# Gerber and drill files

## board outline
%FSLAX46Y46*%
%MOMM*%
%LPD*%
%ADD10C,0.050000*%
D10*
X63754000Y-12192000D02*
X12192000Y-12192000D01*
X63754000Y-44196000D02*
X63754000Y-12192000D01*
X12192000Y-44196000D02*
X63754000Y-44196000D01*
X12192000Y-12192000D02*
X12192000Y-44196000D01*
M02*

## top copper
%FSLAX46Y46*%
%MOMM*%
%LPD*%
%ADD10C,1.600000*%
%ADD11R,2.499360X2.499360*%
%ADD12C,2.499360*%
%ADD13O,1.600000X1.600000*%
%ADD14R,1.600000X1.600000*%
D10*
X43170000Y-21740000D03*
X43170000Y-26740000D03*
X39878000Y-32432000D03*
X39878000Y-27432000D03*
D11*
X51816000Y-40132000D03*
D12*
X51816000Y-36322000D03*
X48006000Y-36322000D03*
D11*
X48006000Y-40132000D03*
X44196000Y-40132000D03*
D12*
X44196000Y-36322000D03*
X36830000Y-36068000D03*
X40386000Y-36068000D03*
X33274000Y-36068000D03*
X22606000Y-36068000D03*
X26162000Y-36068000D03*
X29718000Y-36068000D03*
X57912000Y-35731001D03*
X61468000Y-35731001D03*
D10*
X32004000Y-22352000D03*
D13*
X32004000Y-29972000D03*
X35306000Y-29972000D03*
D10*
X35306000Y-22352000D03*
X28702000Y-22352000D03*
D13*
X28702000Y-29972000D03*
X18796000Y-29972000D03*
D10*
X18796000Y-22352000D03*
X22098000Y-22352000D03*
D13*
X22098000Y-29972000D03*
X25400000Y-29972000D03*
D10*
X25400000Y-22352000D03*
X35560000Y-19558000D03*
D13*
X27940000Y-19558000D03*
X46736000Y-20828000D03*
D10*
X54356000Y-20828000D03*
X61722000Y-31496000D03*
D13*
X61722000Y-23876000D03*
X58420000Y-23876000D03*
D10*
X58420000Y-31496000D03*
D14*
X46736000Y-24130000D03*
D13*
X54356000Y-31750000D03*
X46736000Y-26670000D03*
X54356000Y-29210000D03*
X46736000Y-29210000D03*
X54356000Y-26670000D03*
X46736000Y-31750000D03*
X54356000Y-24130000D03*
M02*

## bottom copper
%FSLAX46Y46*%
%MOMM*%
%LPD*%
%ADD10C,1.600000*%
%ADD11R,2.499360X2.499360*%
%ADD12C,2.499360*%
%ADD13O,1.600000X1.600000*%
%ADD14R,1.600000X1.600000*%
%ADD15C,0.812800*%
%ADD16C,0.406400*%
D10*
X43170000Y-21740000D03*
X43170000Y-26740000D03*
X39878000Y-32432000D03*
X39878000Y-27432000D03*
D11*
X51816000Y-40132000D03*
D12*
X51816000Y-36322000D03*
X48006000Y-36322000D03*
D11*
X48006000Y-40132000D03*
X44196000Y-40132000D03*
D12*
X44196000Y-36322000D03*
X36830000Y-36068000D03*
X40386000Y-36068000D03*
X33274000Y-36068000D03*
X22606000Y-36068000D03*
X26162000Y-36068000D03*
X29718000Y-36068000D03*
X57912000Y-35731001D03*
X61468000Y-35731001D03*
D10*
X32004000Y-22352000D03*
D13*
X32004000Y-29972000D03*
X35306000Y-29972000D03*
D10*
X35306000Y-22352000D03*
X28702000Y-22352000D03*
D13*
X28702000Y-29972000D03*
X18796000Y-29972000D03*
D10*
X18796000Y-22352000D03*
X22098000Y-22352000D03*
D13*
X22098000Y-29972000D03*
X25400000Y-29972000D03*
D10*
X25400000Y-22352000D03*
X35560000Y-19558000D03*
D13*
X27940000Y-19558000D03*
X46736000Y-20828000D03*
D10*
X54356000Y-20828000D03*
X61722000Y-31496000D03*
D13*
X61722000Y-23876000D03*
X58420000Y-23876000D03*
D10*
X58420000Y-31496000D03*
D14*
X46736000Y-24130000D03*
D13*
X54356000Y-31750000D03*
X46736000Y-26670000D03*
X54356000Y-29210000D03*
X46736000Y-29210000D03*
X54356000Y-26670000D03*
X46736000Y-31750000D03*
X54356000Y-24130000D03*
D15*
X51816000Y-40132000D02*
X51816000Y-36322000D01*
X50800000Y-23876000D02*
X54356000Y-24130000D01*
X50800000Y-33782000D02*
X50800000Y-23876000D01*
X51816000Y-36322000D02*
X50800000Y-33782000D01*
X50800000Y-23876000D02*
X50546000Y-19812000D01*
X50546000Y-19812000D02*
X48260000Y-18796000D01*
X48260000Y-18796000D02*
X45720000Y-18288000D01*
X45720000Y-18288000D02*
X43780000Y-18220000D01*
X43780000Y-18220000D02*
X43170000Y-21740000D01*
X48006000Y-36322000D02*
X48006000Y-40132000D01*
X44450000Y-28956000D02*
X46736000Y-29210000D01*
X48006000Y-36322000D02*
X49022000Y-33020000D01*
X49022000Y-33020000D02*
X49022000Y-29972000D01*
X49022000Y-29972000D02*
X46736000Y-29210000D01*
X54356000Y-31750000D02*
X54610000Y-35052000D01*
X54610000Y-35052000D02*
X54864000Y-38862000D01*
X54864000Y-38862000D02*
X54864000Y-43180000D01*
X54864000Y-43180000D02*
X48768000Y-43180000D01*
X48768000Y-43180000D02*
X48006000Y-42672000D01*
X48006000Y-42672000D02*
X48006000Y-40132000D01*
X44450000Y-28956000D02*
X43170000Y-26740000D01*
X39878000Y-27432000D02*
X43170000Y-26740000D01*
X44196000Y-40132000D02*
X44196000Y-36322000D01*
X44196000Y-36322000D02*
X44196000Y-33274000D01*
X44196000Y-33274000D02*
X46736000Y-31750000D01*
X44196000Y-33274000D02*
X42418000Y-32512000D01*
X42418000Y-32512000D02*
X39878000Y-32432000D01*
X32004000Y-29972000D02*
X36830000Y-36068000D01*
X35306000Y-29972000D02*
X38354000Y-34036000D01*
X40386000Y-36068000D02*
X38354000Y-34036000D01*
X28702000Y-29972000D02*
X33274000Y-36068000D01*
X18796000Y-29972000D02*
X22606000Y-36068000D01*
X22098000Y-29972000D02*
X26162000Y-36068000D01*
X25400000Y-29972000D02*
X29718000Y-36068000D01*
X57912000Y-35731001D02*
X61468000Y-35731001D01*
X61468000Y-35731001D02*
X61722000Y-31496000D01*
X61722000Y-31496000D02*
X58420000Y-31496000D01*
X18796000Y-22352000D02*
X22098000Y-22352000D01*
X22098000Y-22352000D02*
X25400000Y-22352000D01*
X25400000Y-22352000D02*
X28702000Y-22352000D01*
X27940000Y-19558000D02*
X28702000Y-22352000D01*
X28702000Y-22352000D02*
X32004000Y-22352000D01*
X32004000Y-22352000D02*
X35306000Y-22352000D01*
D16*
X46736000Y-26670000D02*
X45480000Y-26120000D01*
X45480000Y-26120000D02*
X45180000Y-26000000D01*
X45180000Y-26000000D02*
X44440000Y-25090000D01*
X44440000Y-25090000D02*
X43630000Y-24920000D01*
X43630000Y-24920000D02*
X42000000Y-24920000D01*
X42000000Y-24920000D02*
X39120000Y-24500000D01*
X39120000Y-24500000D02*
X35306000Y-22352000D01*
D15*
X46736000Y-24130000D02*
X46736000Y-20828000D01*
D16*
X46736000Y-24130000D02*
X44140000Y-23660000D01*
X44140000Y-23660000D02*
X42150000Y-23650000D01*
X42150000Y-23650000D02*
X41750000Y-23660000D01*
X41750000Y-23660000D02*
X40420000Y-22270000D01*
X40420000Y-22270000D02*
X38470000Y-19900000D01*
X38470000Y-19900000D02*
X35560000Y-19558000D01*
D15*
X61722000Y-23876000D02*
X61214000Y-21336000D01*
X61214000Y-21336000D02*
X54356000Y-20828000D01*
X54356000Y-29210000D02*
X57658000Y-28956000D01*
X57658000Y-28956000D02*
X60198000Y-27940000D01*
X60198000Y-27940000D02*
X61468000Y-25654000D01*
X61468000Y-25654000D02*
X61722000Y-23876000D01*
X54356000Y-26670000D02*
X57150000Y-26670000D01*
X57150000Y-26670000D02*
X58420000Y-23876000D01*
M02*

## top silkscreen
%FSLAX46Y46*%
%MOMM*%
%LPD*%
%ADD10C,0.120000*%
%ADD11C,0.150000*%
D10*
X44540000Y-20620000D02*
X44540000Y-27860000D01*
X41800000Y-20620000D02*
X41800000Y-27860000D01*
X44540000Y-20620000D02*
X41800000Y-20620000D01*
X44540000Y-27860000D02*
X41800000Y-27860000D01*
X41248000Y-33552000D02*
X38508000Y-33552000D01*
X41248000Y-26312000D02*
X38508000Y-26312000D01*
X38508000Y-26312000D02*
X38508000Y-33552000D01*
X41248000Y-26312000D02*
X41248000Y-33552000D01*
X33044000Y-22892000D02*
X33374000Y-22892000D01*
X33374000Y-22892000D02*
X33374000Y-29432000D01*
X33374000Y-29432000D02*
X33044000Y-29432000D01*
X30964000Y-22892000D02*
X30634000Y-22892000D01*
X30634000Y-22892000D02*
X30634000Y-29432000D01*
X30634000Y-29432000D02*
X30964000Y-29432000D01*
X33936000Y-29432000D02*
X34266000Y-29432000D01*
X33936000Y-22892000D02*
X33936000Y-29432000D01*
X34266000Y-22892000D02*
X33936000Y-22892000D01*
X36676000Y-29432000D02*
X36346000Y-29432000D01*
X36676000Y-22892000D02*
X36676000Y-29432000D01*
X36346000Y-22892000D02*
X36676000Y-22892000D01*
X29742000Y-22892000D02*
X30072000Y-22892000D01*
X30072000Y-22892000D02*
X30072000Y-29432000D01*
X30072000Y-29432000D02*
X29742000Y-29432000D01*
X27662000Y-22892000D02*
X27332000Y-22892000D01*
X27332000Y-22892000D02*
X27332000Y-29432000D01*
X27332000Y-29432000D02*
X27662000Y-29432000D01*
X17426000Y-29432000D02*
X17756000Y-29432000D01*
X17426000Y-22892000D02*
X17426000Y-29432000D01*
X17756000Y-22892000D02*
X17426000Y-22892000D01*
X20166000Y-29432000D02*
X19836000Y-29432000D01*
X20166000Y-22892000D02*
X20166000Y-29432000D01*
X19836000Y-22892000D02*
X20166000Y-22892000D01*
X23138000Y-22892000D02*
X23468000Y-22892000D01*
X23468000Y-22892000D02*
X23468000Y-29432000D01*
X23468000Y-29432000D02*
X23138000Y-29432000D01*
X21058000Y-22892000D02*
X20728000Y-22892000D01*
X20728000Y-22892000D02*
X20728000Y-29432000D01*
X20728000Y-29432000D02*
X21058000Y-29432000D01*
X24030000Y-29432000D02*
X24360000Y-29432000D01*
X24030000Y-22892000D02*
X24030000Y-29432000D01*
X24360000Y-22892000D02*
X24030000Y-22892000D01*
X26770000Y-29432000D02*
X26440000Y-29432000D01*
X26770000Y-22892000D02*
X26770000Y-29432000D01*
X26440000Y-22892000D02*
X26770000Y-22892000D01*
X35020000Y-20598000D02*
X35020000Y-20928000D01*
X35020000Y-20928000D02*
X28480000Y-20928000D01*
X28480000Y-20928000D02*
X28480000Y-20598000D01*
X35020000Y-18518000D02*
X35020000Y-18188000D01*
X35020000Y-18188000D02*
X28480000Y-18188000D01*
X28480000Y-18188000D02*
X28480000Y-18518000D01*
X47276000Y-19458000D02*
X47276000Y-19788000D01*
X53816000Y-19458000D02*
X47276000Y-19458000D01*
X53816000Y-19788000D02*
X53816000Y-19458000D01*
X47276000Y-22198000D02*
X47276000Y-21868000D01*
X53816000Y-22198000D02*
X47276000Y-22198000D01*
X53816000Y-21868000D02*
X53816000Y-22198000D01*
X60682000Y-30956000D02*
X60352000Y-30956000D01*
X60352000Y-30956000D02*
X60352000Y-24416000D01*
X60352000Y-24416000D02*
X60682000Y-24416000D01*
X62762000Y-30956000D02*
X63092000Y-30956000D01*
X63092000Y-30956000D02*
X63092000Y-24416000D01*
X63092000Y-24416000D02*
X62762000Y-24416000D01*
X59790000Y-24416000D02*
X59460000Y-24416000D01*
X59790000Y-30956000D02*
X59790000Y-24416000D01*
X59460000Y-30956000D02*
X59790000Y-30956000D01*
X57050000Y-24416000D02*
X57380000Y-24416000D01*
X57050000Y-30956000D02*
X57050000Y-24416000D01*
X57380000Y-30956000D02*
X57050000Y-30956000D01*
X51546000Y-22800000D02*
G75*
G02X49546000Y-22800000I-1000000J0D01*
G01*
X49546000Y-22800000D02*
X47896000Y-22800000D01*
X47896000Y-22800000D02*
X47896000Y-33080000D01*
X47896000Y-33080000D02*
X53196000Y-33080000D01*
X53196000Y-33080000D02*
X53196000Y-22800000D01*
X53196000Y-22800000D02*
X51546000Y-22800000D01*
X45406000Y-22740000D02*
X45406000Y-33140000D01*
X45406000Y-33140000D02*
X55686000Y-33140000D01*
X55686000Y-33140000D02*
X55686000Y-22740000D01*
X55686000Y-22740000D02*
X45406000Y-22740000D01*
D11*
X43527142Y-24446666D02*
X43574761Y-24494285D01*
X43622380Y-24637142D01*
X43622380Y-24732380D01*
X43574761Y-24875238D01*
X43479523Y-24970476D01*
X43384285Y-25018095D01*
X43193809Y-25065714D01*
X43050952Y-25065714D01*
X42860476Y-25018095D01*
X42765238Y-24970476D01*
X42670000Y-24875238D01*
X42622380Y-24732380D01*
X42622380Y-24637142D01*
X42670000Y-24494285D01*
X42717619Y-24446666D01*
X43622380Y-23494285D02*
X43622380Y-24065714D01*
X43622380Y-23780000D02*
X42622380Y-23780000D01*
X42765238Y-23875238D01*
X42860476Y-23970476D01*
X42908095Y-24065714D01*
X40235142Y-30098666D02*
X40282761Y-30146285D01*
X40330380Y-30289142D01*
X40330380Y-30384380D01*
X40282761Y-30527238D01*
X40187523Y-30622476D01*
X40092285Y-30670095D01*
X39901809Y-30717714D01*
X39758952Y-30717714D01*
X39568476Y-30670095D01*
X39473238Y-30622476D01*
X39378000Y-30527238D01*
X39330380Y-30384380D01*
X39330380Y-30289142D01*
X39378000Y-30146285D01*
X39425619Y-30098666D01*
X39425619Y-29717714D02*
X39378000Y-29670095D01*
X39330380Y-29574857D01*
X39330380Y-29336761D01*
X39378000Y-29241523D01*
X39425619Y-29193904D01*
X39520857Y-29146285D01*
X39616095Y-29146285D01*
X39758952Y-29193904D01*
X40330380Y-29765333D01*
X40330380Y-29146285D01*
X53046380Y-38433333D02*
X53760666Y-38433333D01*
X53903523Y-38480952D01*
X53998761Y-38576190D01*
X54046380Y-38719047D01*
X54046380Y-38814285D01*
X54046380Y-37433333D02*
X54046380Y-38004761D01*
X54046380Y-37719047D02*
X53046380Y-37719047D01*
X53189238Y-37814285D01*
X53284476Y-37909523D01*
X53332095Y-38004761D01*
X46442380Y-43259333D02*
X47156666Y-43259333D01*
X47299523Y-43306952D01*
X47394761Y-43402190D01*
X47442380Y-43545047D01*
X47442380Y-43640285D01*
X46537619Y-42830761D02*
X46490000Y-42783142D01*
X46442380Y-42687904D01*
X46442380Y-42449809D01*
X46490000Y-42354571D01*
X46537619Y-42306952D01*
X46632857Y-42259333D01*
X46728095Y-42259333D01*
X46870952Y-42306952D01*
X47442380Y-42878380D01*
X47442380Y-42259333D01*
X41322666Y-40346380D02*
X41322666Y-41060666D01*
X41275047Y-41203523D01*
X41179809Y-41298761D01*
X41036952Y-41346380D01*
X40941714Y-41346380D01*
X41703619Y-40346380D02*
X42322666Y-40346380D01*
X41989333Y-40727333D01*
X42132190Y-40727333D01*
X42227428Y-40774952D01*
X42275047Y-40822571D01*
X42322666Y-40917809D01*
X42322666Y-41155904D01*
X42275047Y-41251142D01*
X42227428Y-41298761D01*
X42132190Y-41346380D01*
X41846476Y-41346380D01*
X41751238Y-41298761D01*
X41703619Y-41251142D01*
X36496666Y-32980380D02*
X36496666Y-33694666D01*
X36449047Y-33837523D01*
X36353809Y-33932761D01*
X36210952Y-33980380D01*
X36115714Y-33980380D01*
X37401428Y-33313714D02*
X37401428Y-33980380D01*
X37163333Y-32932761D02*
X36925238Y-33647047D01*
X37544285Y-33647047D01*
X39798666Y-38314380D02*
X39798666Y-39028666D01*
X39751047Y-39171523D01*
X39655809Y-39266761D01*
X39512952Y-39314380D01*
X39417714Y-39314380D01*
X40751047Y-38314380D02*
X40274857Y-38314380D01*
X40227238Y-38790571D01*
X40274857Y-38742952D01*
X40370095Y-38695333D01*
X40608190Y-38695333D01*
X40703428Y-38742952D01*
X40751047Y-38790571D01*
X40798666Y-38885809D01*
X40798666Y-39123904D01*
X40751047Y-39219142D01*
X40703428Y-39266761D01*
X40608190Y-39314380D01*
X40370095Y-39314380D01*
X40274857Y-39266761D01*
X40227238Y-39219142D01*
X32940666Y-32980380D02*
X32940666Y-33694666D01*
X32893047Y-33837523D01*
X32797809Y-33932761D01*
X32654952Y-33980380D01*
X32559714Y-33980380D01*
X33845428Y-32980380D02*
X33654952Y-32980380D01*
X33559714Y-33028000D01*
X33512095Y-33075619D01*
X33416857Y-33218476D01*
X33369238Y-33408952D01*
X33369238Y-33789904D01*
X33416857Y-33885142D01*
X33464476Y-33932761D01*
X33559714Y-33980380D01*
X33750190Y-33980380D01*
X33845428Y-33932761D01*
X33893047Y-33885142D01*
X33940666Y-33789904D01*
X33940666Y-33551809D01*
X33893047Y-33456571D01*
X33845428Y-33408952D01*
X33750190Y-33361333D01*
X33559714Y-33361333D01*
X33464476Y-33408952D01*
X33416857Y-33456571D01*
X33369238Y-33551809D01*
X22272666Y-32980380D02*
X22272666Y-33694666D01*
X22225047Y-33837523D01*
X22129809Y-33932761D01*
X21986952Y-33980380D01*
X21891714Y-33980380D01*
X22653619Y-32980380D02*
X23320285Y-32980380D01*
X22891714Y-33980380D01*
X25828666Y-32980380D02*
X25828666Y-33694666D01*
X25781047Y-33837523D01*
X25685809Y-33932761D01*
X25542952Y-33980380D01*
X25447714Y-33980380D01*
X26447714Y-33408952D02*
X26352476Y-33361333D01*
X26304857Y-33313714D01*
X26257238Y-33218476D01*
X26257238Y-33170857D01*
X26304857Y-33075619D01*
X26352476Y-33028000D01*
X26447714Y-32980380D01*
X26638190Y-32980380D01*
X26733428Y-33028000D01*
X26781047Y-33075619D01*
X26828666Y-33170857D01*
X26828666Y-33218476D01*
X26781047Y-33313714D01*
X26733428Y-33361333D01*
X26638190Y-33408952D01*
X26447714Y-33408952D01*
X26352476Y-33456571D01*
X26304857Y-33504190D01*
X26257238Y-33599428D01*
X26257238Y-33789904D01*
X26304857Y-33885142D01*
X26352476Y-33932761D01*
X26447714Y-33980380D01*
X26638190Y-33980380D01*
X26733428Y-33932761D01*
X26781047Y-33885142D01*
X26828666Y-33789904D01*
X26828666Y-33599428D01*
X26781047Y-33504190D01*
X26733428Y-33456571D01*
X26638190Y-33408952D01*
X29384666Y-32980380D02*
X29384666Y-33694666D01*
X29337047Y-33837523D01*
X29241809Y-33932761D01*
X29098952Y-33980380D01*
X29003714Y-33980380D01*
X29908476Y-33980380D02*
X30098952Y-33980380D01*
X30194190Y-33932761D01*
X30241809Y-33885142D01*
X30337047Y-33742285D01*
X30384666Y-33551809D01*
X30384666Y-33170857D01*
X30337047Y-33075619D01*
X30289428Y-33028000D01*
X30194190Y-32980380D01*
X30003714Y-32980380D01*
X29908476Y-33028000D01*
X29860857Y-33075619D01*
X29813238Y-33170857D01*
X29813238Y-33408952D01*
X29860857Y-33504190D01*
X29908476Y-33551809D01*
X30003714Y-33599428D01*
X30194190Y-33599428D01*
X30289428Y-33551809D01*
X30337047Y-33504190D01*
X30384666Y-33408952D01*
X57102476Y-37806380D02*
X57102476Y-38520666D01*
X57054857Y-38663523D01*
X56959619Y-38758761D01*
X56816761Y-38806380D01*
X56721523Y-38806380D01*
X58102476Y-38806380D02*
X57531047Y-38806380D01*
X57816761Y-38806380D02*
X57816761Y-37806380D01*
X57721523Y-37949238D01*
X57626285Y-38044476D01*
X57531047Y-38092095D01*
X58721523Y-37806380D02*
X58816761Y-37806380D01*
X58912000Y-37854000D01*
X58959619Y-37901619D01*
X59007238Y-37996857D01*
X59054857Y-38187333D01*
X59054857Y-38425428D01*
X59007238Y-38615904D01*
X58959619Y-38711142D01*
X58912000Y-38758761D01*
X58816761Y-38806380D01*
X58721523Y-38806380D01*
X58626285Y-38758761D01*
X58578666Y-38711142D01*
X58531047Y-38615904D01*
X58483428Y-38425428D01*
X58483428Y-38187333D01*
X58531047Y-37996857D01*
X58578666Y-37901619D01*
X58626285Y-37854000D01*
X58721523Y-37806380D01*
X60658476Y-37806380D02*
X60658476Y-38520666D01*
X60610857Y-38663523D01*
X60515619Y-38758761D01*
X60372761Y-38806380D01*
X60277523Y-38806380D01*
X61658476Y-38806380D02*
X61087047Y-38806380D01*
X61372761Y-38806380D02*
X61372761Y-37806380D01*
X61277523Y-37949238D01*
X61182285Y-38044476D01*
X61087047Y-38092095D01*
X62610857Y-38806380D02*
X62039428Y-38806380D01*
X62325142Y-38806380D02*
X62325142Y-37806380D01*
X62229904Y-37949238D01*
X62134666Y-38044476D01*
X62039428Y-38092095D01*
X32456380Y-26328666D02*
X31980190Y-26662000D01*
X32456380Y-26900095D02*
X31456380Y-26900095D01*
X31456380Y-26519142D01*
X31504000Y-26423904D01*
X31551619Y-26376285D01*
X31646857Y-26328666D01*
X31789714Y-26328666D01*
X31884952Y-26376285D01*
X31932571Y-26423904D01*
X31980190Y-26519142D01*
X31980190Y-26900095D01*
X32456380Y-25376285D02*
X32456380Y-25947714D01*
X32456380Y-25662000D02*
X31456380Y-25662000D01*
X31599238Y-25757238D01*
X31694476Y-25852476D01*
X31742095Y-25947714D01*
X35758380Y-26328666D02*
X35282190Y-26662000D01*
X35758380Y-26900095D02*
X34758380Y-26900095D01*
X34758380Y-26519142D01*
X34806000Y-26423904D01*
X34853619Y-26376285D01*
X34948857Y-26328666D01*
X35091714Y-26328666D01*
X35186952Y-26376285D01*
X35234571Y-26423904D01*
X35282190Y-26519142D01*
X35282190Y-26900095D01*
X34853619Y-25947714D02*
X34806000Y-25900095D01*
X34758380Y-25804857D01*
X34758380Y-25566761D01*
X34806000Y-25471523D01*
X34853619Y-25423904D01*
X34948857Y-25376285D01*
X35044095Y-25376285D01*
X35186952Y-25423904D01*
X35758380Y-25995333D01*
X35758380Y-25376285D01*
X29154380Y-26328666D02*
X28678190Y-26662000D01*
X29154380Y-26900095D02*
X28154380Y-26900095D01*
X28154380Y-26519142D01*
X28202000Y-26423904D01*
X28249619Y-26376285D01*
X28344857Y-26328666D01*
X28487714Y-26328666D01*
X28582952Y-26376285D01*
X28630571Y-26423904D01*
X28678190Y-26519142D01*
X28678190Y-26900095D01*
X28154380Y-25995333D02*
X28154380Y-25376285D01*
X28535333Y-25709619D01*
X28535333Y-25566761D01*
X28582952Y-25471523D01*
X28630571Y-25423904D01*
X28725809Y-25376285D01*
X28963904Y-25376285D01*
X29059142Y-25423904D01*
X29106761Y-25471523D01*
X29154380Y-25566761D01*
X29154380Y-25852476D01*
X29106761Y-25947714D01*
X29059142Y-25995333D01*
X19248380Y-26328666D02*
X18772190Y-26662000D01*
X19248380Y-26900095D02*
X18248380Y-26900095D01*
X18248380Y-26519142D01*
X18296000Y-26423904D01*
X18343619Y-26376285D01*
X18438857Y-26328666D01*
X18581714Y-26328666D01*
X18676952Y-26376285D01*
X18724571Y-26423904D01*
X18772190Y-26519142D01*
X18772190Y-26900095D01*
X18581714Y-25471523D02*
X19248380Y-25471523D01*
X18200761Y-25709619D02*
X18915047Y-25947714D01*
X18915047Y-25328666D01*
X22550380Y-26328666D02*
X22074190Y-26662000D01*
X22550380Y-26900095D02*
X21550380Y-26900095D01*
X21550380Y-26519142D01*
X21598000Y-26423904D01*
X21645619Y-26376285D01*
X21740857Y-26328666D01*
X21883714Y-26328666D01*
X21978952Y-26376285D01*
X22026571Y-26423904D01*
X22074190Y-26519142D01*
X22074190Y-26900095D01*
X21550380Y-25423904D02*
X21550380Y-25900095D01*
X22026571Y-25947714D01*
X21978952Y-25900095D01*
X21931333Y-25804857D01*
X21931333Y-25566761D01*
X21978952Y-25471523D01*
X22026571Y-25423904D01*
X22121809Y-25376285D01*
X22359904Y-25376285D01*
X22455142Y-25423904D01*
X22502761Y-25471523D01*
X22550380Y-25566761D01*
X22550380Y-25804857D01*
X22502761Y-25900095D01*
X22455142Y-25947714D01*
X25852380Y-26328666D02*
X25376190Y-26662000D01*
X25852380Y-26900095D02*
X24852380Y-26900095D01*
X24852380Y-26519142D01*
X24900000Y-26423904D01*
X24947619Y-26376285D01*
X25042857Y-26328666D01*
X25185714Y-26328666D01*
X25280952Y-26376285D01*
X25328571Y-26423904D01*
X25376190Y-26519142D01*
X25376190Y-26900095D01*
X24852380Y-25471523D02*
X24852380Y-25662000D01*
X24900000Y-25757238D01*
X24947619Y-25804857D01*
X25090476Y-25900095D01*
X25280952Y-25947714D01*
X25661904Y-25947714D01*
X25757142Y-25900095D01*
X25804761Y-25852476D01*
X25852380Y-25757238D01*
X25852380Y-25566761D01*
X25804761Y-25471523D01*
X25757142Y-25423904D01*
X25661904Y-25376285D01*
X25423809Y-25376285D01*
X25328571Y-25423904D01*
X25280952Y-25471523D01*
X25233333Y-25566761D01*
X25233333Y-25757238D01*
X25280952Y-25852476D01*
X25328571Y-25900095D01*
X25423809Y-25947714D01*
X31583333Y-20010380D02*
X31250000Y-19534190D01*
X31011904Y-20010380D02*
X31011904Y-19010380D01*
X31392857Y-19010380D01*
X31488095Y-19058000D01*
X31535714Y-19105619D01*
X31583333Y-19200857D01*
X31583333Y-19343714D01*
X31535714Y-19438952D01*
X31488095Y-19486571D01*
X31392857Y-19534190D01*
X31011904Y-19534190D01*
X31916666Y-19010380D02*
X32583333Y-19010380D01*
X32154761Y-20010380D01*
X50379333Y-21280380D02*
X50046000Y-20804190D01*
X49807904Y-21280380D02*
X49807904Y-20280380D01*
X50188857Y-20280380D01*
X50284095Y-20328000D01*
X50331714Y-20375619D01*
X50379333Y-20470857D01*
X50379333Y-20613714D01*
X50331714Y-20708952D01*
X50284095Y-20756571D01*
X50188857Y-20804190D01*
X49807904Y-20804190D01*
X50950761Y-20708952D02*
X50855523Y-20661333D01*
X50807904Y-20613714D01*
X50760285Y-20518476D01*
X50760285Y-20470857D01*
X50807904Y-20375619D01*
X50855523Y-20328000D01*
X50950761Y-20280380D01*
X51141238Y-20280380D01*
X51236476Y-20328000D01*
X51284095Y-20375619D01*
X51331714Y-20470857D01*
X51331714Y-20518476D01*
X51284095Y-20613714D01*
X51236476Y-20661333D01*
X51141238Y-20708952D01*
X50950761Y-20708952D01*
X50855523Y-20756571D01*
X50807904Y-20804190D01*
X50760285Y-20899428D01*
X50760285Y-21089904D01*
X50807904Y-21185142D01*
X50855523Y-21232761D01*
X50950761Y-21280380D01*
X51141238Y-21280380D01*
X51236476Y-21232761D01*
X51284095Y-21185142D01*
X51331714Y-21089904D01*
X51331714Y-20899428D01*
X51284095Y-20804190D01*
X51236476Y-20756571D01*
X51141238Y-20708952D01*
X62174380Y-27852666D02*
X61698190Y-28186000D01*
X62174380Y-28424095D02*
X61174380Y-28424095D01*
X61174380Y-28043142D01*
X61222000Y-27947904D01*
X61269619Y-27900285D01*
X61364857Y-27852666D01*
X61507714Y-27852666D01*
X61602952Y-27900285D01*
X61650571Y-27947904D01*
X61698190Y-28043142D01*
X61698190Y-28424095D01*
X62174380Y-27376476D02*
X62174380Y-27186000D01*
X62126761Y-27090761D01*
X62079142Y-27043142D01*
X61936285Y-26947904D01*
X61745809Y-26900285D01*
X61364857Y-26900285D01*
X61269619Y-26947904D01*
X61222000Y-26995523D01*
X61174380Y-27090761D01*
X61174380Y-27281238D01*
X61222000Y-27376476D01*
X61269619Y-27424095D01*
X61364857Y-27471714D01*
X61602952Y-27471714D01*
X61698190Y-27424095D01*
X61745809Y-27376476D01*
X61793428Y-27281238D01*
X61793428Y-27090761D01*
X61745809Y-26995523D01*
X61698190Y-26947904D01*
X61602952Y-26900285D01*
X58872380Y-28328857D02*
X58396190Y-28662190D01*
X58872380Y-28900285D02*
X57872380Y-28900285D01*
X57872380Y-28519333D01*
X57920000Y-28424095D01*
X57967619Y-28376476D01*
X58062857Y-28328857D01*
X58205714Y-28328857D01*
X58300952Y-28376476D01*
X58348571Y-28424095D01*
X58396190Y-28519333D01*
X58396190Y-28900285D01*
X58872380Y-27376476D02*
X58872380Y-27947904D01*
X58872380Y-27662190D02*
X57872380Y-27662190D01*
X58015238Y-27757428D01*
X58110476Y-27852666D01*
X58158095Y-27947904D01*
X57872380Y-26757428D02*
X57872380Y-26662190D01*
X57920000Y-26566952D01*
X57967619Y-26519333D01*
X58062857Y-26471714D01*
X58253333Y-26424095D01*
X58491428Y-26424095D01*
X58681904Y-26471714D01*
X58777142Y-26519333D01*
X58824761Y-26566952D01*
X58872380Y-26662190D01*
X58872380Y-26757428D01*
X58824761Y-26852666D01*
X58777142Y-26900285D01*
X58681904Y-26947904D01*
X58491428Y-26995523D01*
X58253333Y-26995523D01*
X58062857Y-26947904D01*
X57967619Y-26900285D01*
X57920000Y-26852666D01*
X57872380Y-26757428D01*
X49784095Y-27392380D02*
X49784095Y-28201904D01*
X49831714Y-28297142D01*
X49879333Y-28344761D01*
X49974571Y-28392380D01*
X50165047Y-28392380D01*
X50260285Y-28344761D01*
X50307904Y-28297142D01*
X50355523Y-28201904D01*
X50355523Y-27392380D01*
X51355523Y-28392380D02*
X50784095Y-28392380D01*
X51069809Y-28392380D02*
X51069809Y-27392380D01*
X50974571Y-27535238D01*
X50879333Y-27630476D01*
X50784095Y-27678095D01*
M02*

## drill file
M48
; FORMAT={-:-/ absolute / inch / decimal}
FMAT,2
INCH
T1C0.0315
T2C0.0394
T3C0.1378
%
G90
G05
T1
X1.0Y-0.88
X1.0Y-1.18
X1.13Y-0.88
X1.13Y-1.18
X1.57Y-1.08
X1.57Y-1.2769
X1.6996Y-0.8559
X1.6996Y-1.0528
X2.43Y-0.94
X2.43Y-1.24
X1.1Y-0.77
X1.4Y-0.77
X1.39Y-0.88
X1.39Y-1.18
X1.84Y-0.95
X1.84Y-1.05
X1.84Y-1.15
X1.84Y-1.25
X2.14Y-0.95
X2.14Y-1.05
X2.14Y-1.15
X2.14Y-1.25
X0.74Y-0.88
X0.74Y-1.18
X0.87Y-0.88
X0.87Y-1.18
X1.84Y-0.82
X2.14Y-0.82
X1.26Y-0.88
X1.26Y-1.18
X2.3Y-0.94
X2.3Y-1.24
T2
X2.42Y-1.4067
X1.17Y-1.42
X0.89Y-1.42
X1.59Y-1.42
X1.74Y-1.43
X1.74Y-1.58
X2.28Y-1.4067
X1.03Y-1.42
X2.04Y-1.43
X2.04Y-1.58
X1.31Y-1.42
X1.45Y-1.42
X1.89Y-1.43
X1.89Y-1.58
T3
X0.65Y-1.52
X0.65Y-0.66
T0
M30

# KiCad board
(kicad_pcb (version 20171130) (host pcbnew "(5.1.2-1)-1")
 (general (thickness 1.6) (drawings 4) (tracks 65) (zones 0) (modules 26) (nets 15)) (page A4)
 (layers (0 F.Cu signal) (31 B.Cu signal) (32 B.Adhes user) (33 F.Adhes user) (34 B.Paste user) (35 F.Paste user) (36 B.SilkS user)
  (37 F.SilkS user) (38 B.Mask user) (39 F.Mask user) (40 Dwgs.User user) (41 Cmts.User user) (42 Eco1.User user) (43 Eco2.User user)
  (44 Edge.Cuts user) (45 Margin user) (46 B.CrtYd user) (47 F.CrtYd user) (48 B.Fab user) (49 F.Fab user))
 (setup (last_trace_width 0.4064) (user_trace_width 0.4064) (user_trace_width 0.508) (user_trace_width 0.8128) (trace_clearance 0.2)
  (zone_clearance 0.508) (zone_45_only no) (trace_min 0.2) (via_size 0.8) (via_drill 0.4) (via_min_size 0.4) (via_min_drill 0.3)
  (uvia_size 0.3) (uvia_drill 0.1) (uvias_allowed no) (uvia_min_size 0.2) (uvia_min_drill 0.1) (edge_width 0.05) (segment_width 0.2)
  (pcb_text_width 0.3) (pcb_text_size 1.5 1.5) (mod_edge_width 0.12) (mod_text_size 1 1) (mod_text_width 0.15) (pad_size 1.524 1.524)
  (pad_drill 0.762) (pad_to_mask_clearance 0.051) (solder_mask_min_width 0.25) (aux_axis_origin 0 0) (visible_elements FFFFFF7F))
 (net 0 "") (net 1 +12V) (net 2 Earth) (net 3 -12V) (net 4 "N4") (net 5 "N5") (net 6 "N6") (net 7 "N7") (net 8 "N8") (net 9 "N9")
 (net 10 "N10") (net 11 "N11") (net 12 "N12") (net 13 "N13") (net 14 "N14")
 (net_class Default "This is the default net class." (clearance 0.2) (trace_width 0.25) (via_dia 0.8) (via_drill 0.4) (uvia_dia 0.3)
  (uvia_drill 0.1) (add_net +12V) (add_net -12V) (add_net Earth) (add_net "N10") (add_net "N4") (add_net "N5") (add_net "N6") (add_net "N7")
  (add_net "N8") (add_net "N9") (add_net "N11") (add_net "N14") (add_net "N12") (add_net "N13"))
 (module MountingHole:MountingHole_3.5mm (layer F.Cu) (at 16.51 38.608)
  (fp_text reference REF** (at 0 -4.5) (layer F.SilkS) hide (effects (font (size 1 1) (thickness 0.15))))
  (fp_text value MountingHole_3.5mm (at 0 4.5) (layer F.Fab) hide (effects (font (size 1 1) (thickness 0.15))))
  (pad 1 np_thru_hole circle (at 0 0) (size 3.5 3.5) (drill 3.5) (layers *.Cu *.Mask)))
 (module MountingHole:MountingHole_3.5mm (layer F.Cu) (at 16.51 16.764)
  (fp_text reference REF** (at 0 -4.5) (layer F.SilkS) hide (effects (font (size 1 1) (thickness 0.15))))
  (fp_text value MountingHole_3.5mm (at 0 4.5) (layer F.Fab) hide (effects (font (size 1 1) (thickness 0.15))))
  (pad 1 np_thru_hole circle (at 0 0) (size 3.5 3.5) (drill 3.5) (layers *.Cu *.Mask)))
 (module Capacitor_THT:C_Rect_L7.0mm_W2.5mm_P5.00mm (layer F.Cu) (at 43.17 21.74 270)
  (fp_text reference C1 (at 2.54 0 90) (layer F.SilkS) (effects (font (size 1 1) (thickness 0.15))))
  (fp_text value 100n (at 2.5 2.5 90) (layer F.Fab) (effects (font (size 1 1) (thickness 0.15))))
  (fp_line (start -1.12 -1.37) (end 6.12 -1.37) (layer F.SilkS) (width 0.12))
  (fp_line (start -1.12 1.37) (end 6.12 1.37) (layer F.SilkS) (width 0.12))
  (fp_line (start -1.12 -1.37) (end -1.12 1.37) (layer F.SilkS) (width 0.12))
  (fp_line (start 6.12 -1.37) (end 6.12 1.37) (layer F.SilkS) (width 0.12))
  (pad 1 thru_hole circle (at 0 0 270) (size 1.6 1.6) (drill 0.8) (layers *.Cu *.Mask) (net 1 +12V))
  (pad 2 thru_hole circle (at 5 0 270) (size 1.6 1.6) (drill 0.8) (layers *.Cu *.Mask) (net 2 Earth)))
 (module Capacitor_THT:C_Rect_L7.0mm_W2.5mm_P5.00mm (layer F.Cu) (at 39.878 27.432 270)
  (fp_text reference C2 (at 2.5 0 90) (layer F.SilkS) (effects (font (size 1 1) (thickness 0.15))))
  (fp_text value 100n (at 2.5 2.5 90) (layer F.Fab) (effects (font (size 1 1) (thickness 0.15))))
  (fp_line (start 6.12 -1.37) (end 6.12 1.37) (layer F.SilkS) (width 0.12))
  (fp_line (start -1.12 -1.37) (end -1.12 1.37) (layer F.SilkS) (width 0.12))
  (fp_line (start -1.12 1.37) (end 6.12 1.37) (layer F.SilkS) (width 0.12))
  (fp_line (start -1.12 -1.37) (end 6.12 -1.37) (layer F.SilkS) (width 0.12))
  (pad 2 thru_hole circle (at 5 0 270) (size 1.6 1.6) (drill 0.8) (layers *.Cu *.Mask) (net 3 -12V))
  (pad 1 thru_hole circle (at 0 0 270) (size 1.6 1.6) (drill 0.8) (layers *.Cu *.Mask) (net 2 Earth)))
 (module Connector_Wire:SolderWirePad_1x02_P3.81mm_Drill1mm (layer F.Cu) (at 51.816 40.132 90)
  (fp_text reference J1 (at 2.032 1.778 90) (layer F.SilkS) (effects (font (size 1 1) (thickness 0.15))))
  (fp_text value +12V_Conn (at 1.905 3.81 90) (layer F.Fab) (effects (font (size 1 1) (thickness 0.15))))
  (pad 1 thru_hole rect (at 0 0 90) (size 2.49936 2.49936) (drill 1.00076) (layers *.Cu *.Mask) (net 1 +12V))
  (pad 2 thru_hole circle (at 3.81 0 90) (size 2.49936 2.49936) (drill 1.00076) (layers *.Cu *.Mask) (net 1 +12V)))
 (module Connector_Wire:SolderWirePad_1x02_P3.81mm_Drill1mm (layer F.Cu) (at 48.006 40.132 90)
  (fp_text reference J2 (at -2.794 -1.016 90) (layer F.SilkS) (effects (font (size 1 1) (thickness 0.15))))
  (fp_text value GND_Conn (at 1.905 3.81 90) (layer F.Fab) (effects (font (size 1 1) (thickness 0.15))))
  (pad 2 thru_hole circle (at 3.81 0 90) (size 2.49936 2.49936) (drill 1.00076) (layers *.Cu *.Mask) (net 2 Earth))
  (pad 1 thru_hole rect (at 0 0 90) (size 2.49936 2.49936) (drill 1.00076) (layers *.Cu *.Mask) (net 2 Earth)))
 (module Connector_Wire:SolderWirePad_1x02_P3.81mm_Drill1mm (layer F.Cu) (at 44.196 40.132 90)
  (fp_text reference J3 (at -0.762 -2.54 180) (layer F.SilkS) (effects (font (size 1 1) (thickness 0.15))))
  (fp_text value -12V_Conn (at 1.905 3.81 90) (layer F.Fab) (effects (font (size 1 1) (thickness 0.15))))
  (pad 1 thru_hole rect (at 0 0 90) (size 2.49936 2.49936) (drill 1.00076) (layers *.Cu *.Mask) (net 3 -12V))
  (pad 2 thru_hole circle (at 3.81 0 90) (size 2.49936 2.49936) (drill 1.00076) (layers *.Cu *.Mask) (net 3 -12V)))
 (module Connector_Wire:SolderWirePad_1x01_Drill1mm (layer F.Cu) (at 36.83 36.068)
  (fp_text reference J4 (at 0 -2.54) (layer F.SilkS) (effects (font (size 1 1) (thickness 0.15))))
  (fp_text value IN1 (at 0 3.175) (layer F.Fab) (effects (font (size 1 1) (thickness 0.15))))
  (pad 1 thru_hole circle (at 0 0) (size 2.49936 2.49936) (drill 1.00076) (layers *.Cu *.Mask) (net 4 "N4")))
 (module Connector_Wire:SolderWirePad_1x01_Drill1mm (layer F.Cu) (at 40.386 36.068)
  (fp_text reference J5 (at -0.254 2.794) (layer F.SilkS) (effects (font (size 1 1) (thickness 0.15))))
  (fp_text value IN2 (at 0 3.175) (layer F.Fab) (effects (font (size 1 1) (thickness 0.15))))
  (pad 1 thru_hole circle (at 0 0) (size 2.49936 2.49936) (drill 1.00076) (layers *.Cu *.Mask) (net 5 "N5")))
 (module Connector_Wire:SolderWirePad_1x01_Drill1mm (layer F.Cu) (at 33.274 36.068)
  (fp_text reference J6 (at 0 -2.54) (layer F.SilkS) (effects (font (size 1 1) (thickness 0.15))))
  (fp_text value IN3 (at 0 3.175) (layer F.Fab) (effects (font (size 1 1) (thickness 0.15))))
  (pad 1 thru_hole circle (at 0 0) (size 2.49936 2.49936) (drill 1.00076) (layers *.Cu *.Mask) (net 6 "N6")))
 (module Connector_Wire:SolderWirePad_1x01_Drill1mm (layer F.Cu) (at 22.606 36.068)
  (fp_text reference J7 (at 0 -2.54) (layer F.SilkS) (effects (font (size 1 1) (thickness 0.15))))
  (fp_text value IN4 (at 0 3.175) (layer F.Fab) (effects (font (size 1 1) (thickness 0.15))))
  (pad 1 thru_hole circle (at 0 0) (size 2.49936 2.49936) (drill 1.00076) (layers *.Cu *.Mask) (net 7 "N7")))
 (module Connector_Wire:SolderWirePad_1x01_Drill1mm (layer F.Cu) (at 26.162 36.068)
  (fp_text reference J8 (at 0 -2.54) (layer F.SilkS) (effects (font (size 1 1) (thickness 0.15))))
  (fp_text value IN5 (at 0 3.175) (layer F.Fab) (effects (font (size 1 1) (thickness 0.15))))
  (pad 1 thru_hole circle (at 0 0) (size 2.49936 2.49936) (drill 1.00076) (layers *.Cu *.Mask) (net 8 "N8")))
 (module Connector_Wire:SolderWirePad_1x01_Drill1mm (layer F.Cu) (at 29.718 36.068)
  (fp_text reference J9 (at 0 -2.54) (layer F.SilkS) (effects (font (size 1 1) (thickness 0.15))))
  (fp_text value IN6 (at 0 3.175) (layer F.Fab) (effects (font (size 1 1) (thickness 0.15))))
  (pad 1 thru_hole circle (at 0 0) (size 2.49936 2.49936) (drill 1.00076) (layers *.Cu *.Mask) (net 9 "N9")))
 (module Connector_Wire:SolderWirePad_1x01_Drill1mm (layer F.Cu) (at 57.912 35.731001)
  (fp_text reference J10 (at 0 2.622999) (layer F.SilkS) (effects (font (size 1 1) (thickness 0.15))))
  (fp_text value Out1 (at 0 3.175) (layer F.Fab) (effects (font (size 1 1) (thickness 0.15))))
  (pad 1 thru_hole circle (at 0 0) (size 2.49936 2.49936) (drill 1.00076) (layers *.Cu *.Mask) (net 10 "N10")))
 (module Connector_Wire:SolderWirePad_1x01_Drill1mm (layer F.Cu) (at 61.468 35.731001)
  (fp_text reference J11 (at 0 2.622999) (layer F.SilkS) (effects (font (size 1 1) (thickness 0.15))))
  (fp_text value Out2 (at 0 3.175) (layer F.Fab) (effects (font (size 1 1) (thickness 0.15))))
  (pad 1 thru_hole circle (at 0 0) (size 2.49936 2.49936) (drill 1.00076) (layers *.Cu *.Mask) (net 10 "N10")))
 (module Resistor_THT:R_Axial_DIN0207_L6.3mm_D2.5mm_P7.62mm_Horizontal (layer F.Cu) (at 32.004 22.352 270)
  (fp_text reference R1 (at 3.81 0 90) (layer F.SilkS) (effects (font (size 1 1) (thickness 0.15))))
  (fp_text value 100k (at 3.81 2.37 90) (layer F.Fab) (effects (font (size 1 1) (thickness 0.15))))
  (fp_line (start 0.54 -1.04) (end 0.54 -1.37) (layer F.SilkS) (width 0.12))
  (fp_line (start 0.54 -1.37) (end 7.08 -1.37) (layer F.SilkS) (width 0.12))
  (fp_line (start 7.08 -1.37) (end 7.08 -1.04) (layer F.SilkS) (width 0.12))
  (fp_line (start 0.54 1.04) (end 0.54 1.37) (layer F.SilkS) (width 0.12))
  (fp_line (start 0.54 1.37) (end 7.08 1.37) (layer F.SilkS) (width 0.12))
  (fp_line (start 7.08 1.37) (end 7.08 1.04) (layer F.SilkS) (width 0.12))
  (pad 1 thru_hole circle (at 0 0 270) (size 1.6 1.6) (drill 0.8) (layers *.Cu *.Mask) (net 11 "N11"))
  (pad 2 thru_hole oval (at 7.62 0 270) (size 1.6 1.6) (drill 0.8) (layers *.Cu *.Mask) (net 4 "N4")))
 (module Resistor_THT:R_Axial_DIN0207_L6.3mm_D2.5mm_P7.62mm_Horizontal (layer F.Cu) (at 35.306 22.352 270)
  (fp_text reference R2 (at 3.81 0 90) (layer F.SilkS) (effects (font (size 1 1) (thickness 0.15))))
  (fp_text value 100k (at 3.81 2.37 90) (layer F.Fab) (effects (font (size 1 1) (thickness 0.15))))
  (fp_line (start 7.08 1.37) (end 7.08 1.04) (layer F.SilkS) (width 0.12))
  (fp_line (start 0.54 1.37) (end 7.08 1.37) (layer F.SilkS) (width 0.12))
  (fp_line (start 0.54 1.04) (end 0.54 1.37) (layer F.SilkS) (width 0.12))
  (fp_line (start 7.08 -1.37) (end 7.08 -1.04) (layer F.SilkS) (width 0.12))
  (fp_line (start 0.54 -1.37) (end 7.08 -1.37) (layer F.SilkS) (width 0.12))
  (fp_line (start 0.54 -1.04) (end 0.54 -1.37) (layer F.SilkS) (width 0.12))
  (pad 2 thru_hole oval (at 7.62 0 270) (size 1.6 1.6) (drill 0.8) (layers *.Cu *.Mask) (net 5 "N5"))
  (pad 1 thru_hole circle (at 0 0 270) (size 1.6 1.6) (drill 0.8) (layers *.Cu *.Mask) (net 11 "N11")))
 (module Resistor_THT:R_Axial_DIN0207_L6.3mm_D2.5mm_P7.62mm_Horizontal (layer F.Cu) (at 28.702 22.352 270)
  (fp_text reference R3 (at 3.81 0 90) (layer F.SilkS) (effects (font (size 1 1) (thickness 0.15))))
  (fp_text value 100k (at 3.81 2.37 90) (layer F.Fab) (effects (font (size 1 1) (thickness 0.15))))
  (fp_line (start 0.54 -1.04) (end 0.54 -1.37) (layer F.SilkS) (width 0.12))
  (fp_line (start 0.54 -1.37) (end 7.08 -1.37) (layer F.SilkS) (width 0.12))
  (fp_line (start 7.08 -1.37) (end 7.08 -1.04) (layer F.SilkS) (width 0.12))
  (fp_line (start 0.54 1.04) (end 0.54 1.37) (layer F.SilkS) (width 0.12))
  (fp_line (start 0.54 1.37) (end 7.08 1.37) (layer F.SilkS) (width 0.12))
  (fp_line (start 7.08 1.37) (end 7.08 1.04) (layer F.SilkS) (width 0.12))
  (pad 1 thru_hole circle (at 0 0 270) (size 1.6 1.6) (drill 0.8) (layers *.Cu *.Mask) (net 11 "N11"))
  (pad 2 thru_hole oval (at 7.62 0 270) (size 1.6 1.6) (drill 0.8) (layers *.Cu *.Mask) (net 6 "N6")))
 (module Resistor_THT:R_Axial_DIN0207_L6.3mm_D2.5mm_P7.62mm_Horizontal (layer F.Cu) (at 18.796 22.352 270)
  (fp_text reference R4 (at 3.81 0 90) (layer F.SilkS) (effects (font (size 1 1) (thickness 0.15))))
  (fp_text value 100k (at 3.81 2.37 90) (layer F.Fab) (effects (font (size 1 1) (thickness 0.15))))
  (fp_line (start 7.08 1.37) (end 7.08 1.04) (layer F.SilkS) (width 0.12))
  (fp_line (start 0.54 1.37) (end 7.08 1.37) (layer F.SilkS) (width 0.12))
  (fp_line (start 0.54 1.04) (end 0.54 1.37) (layer F.SilkS) (width 0.12))
  (fp_line (start 7.08 -1.37) (end 7.08 -1.04) (layer F.SilkS) (width 0.12))
  (fp_line (start 0.54 -1.37) (end 7.08 -1.37) (layer F.SilkS) (width 0.12))
  (fp_line (start 0.54 -1.04) (end 0.54 -1.37) (layer F.SilkS) (width 0.12))
  (pad 2 thru_hole oval (at 7.62 0 270) (size 1.6 1.6) (drill 0.8) (layers *.Cu *.Mask) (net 7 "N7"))
  (pad 1 thru_hole circle (at 0 0 270) (size 1.6 1.6) (drill 0.8) (layers *.Cu *.Mask) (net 11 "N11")))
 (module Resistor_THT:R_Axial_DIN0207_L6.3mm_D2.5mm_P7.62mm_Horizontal (layer F.Cu) (at 22.098 22.352 270)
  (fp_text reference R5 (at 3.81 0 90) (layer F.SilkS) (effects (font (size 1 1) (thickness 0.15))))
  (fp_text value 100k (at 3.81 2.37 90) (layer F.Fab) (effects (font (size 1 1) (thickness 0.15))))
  (fp_line (start 0.54 -1.04) (end 0.54 -1.37) (layer F.SilkS) (width 0.12))
  (fp_line (start 0.54 -1.37) (end 7.08 -1.37) (layer F.SilkS) (width 0.12))
  (fp_line (start 7.08 -1.37) (end 7.08 -1.04) (layer F.SilkS) (width 0.12))
  (fp_line (start 0.54 1.04) (end 0.54 1.37) (layer F.SilkS) (width 0.12))
  (fp_line (start 0.54 1.37) (end 7.08 1.37) (layer F.SilkS) (width 0.12))
  (fp_line (start 7.08 1.37) (end 7.08 1.04) (layer F.SilkS) (width 0.12))
  (pad 1 thru_hole circle (at 0 0 270) (size 1.6 1.6) (drill 0.8) (layers *.Cu *.Mask) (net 11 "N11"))
  (pad 2 thru_hole oval (at 7.62 0 270) (size 1.6 1.6) (drill 0.8) (layers *.Cu *.Mask) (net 8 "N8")))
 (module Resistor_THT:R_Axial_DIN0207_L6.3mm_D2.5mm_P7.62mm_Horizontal (layer F.Cu) (at 25.4 22.352 270)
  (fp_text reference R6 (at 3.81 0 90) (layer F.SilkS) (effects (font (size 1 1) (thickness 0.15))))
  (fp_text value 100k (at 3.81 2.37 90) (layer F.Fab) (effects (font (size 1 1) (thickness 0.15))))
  (fp_line (start 7.08 1.37) (end 7.08 1.04) (layer F.SilkS) (width 0.12))
  (fp_line (start 0.54 1.37) (end 7.08 1.37) (layer F.SilkS) (width 0.12))
  (fp_line (start 0.54 1.04) (end 0.54 1.37) (layer F.SilkS) (width 0.12))
  (fp_line (start 7.08 -1.37) (end 7.08 -1.04) (layer F.SilkS) (width 0.12))
  (fp_line (start 0.54 -1.37) (end 7.08 -1.37) (layer F.SilkS) (width 0.12))
  (fp_line (start 0.54 -1.04) (end 0.54 -1.37) (layer F.SilkS) (width 0.12))
  (pad 2 thru_hole oval (at 7.62 0 270) (size 1.6 1.6) (drill 0.8) (layers *.Cu *.Mask) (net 9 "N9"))
  (pad 1 thru_hole circle (at 0 0 270) (size 1.6 1.6) (drill 0.8) (layers *.Cu *.Mask) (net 11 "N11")))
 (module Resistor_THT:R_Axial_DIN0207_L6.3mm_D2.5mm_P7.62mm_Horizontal (layer F.Cu) (at 35.56 19.558 180)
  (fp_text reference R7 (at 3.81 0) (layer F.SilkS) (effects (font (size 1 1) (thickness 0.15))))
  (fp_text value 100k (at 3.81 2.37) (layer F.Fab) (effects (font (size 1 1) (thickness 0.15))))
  (fp_line (start 0.54 -1.04) (end 0.54 -1.37) (layer F.SilkS) (width 0.12))
  (fp_line (start 0.54 -1.37) (end 7.08 -1.37) (layer F.SilkS) (width 0.12))
  (fp_line (start 7.08 -1.37) (end 7.08 -1.04) (layer F.SilkS) (width 0.12))
  (fp_line (start 0.54 1.04) (end 0.54 1.37) (layer F.SilkS) (width 0.12))
  (fp_line (start 0.54 1.37) (end 7.08 1.37) (layer F.SilkS) (width 0.12))
  (fp_line (start 7.08 1.37) (end 7.08 1.04) (layer F.SilkS) (width 0.12))
  (pad 1 thru_hole circle (at 0 0 180) (size 1.6 1.6) (drill 0.8) (layers *.Cu *.Mask) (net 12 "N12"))
  (pad 2 thru_hole oval (at 7.62 0 180) (size 1.6 1.6) (drill 0.8) (layers *.Cu *.Mask) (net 11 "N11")))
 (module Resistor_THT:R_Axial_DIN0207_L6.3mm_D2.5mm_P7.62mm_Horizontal (layer F.Cu) (at 54.356 20.828 180)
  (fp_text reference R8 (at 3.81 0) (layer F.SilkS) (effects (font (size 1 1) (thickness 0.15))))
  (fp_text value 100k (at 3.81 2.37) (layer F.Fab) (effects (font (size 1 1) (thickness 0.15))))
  (fp_line (start 7.08 1.37) (end 7.08 1.04) (layer F.SilkS) (width 0.12))
  (fp_line (start 0.54 1.37) (end 7.08 1.37) (layer F.SilkS) (width 0.12))
  (fp_line (start 0.54 1.04) (end 0.54 1.37) (layer F.SilkS) (width 0.12))
  (fp_line (start 7.08 -1.37) (end 7.08 -1.04) (layer F.SilkS) (width 0.12))
  (fp_line (start 0.54 -1.37) (end 7.08 -1.37) (layer F.SilkS) (width 0.12))
  (fp_line (start 0.54 -1.04) (end 0.54 -1.37) (layer F.SilkS) (width 0.12))
  (pad 2 thru_hole oval (at 7.62 0 180) (size 1.6 1.6) (drill 0.8) (layers *.Cu *.Mask) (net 12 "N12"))
  (pad 1 thru_hole circle (at 0 0 180) (size 1.6 1.6) (drill 0.8) (layers *.Cu *.Mask) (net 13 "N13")))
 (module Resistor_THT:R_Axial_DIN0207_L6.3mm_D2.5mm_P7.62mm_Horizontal (layer F.Cu) (at 61.722 31.496 90)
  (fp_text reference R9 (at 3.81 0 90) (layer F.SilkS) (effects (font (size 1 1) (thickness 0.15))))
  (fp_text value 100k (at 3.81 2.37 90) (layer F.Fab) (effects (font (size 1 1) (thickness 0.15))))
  (fp_line (start 0.54 -1.04) (end 0.54 -1.37) (layer F.SilkS) (width 0.12))
  (fp_line (start 0.54 -1.37) (end 7.08 -1.37) (layer F.SilkS) (width 0.12))
  (fp_line (start 7.08 -1.37) (end 7.08 -1.04) (layer F.SilkS) (width 0.12))
  (fp_line (start 0.54 1.04) (end 0.54 1.37) (layer F.SilkS) (width 0.12))
  (fp_line (start 0.54 1.37) (end 7.08 1.37) (layer F.SilkS) (width 0.12))
  (fp_line (start 7.08 1.37) (end 7.08 1.04) (layer F.SilkS) (width 0.12))
  (pad 1 thru_hole circle (at 0 0 90) (size 1.6 1.6) (drill 0.8) (layers *.Cu *.Mask) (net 10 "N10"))
  (pad 2 thru_hole oval (at 7.62 0 90) (size 1.6 1.6) (drill 0.8) (layers *.Cu *.Mask) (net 13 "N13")))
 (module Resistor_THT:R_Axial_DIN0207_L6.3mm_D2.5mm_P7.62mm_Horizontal (layer F.Cu) (at 58.42 31.496 90)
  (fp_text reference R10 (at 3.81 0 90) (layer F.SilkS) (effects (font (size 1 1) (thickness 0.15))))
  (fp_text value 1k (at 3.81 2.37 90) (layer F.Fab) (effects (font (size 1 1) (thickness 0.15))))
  (fp_line (start 7.08 1.37) (end 7.08 1.04) (layer F.SilkS) (width 0.12))
  (fp_line (start 0.54 1.37) (end 7.08 1.37) (layer F.SilkS) (width 0.12))
  (fp_line (start 0.54 1.04) (end 0.54 1.37) (layer F.SilkS) (width 0.12))
  (fp_line (start 7.08 -1.37) (end 7.08 -1.04) (layer F.SilkS) (width 0.12))
  (fp_line (start 0.54 -1.37) (end 7.08 -1.37) (layer F.SilkS) (width 0.12))
  (fp_line (start 0.54 -1.04) (end 0.54 -1.37) (layer F.SilkS) (width 0.12))
  (pad 2 thru_hole oval (at 7.62 0 90) (size 1.6 1.6) (drill 0.8) (layers *.Cu *.Mask) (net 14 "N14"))
  (pad 1 thru_hole circle (at 0 0 90) (size 1.6 1.6) (drill 0.8) (layers *.Cu *.Mask) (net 10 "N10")))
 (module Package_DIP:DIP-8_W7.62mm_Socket (layer F.Cu) (at 46.736 24.13)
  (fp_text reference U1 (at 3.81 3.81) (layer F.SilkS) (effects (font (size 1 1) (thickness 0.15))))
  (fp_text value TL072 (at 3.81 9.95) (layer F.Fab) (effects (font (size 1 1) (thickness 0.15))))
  (fp_arc (start 3.81 -1.33) (end 2.81 -1.33) (angle -180) (layer F.SilkS) (width 0.12))
  (fp_line (start 2.81 -1.33) (end 1.16 -1.33) (layer F.SilkS) (width 0.12))
  (fp_line (start 1.16 -1.33) (end 1.16 8.95) (layer F.SilkS) (width 0.12))
  (fp_line (start 1.16 8.95) (end 6.46 8.95) (layer F.SilkS) (width 0.12))
  (fp_line (start 6.46 8.95) (end 6.46 -1.33) (layer F.SilkS) (width 0.12))
  (fp_line (start 6.46 -1.33) (end 4.81 -1.33) (layer F.SilkS) (width 0.12))
  (fp_line (start -1.33 -1.39) (end -1.33 9.01) (layer F.SilkS) (width 0.12))
  (fp_line (start -1.33 9.01) (end 8.95 9.01) (layer F.SilkS) (width 0.12))
  (fp_line (start 8.95 9.01) (end 8.95 -1.39) (layer F.SilkS) (width 0.12))
  (fp_line (start 8.95 -1.39) (end -1.33 -1.39) (layer F.SilkS) (width 0.12))
  (pad 1 thru_hole rect (at 0 0) (size 1.6 1.6) (drill 0.8) (layers *.Cu *.Mask) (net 12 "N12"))
  (pad 5 thru_hole oval (at 7.62 7.62) (size 1.6 1.6) (drill 0.8) (layers *.Cu *.Mask) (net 2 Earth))
  (pad 2 thru_hole oval (at 0 2.54) (size 1.6 1.6) (drill 0.8) (layers *.Cu *.Mask) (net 11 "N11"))
  (pad 6 thru_hole oval (at 7.62 5.08) (size 1.6 1.6) (drill 0.8) (layers *.Cu *.Mask) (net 13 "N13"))
  (pad 3 thru_hole oval (at 0 5.08) (size 1.6 1.6) (drill 0.8) (layers *.Cu *.Mask) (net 2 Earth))
  (pad 7 thru_hole oval (at 7.62 2.54) (size 1.6 1.6) (drill 0.8) (layers *.Cu *.Mask) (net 14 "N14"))
  (pad 4 thru_hole oval (at 0 7.62) (size 1.6 1.6) (drill 0.8) (layers *.Cu *.Mask) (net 3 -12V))
  (pad 8 thru_hole oval (at 7.62 0) (size 1.6 1.6) (drill 0.8) (layers *.Cu *.Mask) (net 1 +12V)))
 (gr_line (start 63.754 12.192) (end 12.192 12.192) (layer Edge.Cuts) (width 0.05))
 (gr_line (start 63.754 44.196) (end 63.754 12.192) (layer Edge.Cuts) (width 0.05))
 (gr_line (start 12.192 44.196) (end 63.754 44.196) (layer Edge.Cuts) (width 0.05))
 (gr_line (start 12.192 12.192) (end 12.192 44.196) (layer Edge.Cuts) (width 0.05))
 (segment (start 51.816 40.132) (end 51.816 36.322) (width 0.8128) (layer B.Cu) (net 1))
 (segment (start 50.8 23.876) (end 54.356 24.13) (width 0.8128) (layer B.Cu) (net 1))
 (segment (start 50.8 33.782) (end 50.8 23.876) (width 0.8128) (layer B.Cu) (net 1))
 (segment (start 51.816 36.322) (end 50.8 33.782) (width 0.8128) (layer B.Cu) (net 1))
 (segment (start 50.8 23.876) (end 50.546 19.812) (width 0.8128) (layer B.Cu) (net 1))
 (segment (start 50.546 19.812) (end 48.26 18.796) (width 0.8128) (layer B.Cu) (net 1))
 (segment (start 48.26 18.796) (end 45.72 18.288) (width 0.8128) (layer B.Cu) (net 1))
 (segment (start 45.72 18.288) (end 43.78 18.22) (width 0.8128) (layer B.Cu) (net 1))
 (segment (start 43.78 18.22) (end 43.17 21.74) (width 0.8128) (layer B.Cu) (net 1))
 (segment (start 48.006 36.322) (end 48.006 40.132) (width 0.8128) (layer B.Cu) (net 2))
 (segment (start 44.45 28.956) (end 46.736 29.21) (width 0.8128) (layer B.Cu) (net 2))
 (segment (start 48.006 36.322) (end 49.022 33.02) (width 0.8128) (layer B.Cu) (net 2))
 (segment (start 49.022 33.02) (end 49.022 29.972) (width 0.8128) (layer B.Cu) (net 2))
 (segment (start 49.022 29.972) (end 46.736 29.21) (width 0.8128) (layer B.Cu) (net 2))
 (segment (start 54.356 31.75) (end 54.61 35.052) (width 0.8128) (layer B.Cu) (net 2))
 (segment (start 54.61 35.052) (end 54.864 38.862) (width 0.8128) (layer B.Cu) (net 2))
 (segment (start 54.864 38.862) (end 54.864 43.18) (width 0.8128) (layer B.Cu) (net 2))
 (segment (start 54.864 43.18) (end 48.768 43.18) (width 0.8128) (layer B.Cu) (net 2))
 (segment (start 48.768 43.18) (end 48.006 42.672) (width 0.8128) (layer B.Cu) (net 2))
 (segment (start 48.006 42.672) (end 48.006 40.132) (width 0.8128) (layer B.Cu) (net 2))
 (segment (start 44.45 28.956) (end 43.17 26.74) (width 0.8128) (layer B.Cu) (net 2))
 (segment (start 39.878 27.432) (end 43.17 26.74) (width 0.8128) (layer B.Cu) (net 2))
 (segment (start 44.196 40.132) (end 44.196 36.322) (width 0.8128) (layer B.Cu) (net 3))
 (segment (start 44.196 36.322) (end 44.196 33.274) (width 0.8128) (layer B.Cu) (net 3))
 (segment (start 44.196 33.274) (end 46.736 31.75) (width 0.8128) (layer B.Cu) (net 3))
 (segment (start 44.196 33.274) (end 42.418 32.512) (width 0.8128) (layer B.Cu) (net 3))
 (segment (start 42.418 32.512) (end 39.878 32.432) (width 0.8128) (layer B.Cu) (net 3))
 (segment (start 32.004 29.972) (end 36.83 36.068) (width 0.8128) (layer B.Cu) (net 4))
 (segment (start 35.306 29.972) (end 38.354 34.036) (width 0.8128) (layer B.Cu) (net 5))
 (segment (start 40.386 36.068) (end 38.354 34.036) (width 0.8128) (layer B.Cu) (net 5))
 (segment (start 28.702 29.972) (end 33.274 36.068) (width 0.8128) (layer B.Cu) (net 6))
 (segment (start 18.796 29.972) (end 22.606 36.068) (width 0.8128) (layer B.Cu) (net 7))
 (segment (start 22.098 29.972) (end 26.162 36.068) (width 0.8128) (layer B.Cu) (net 8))
 (segment (start 25.4 29.972) (end 29.718 36.068) (width 0.8128) (layer B.Cu) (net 9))
 (segment (start 57.912 35.731001) (end 61.468 35.731001) (width 0.8128) (layer B.Cu) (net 10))
 (segment (start 61.468 35.731001) (end 61.722 31.496) (width 0.8128) (layer B.Cu) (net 10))
 (segment (start 61.722 31.496) (end 58.42 31.496) (width 0.8128) (layer B.Cu) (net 10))
 (segment (start 18.796 22.352) (end 22.098 22.352) (width 0.8128) (layer B.Cu) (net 11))
 (segment (start 22.098 22.352) (end 25.4 22.352) (width 0.8128) (layer B.Cu) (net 11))
 (segment (start 25.4 22.352) (end 28.702 22.352) (width 0.8128) (layer B.Cu) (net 11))
 (segment (start 27.94 19.558) (end 28.702 22.352) (width 0.8128) (layer B.Cu) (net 11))
 (segment (start 28.702 22.352) (end 32.004 22.352) (width 0.8128) (layer B.Cu) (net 11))
 (segment (start 32.004 22.352) (end 35.306 22.352) (width 0.8128) (layer B.Cu) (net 11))
 (segment (start 46.736 26.67) (end 45.48 26.12) (width 0.4064) (layer B.Cu) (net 11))
 (segment (start 45.48 26.12) (end 45.18 26) (width 0.4064) (layer B.Cu) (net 11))
 (segment (start 45.18 26) (end 44.44 25.09) (width 0.4064) (layer B.Cu) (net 11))
 (segment (start 44.44 25.09) (end 43.63 24.92) (width 0.4064) (layer B.Cu) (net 11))
 (segment (start 43.63 24.92) (end 42 24.92) (width 0.4064) (layer B.Cu) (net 11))
 (segment (start 42 24.92) (end 39.12 24.5) (width 0.4064) (layer B.Cu) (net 11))
 (segment (start 39.12 24.5) (end 35.306 22.352) (width 0.4064) (layer B.Cu) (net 11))
 (segment (start 46.736 24.13) (end 46.736 20.828) (width 0.8128) (layer B.Cu) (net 12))
 (segment (start 46.736 24.13) (end 44.14 23.66) (width 0.4064) (layer B.Cu) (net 12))
 (segment (start 44.14 23.66) (end 42.15 23.65) (width 0.4064) (layer B.Cu) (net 12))
 (segment (start 42.15 23.65) (end 41.75 23.66) (width 0.4064) (layer B.Cu) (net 12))
 (segment (start 41.75 23.66) (end 40.42 22.27) (width 0.4064) (layer B.Cu) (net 12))
 (segment (start 40.42 22.27) (end 38.47 19.9) (width 0.4064) (layer B.Cu) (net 12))
 (segment (start 38.47 19.9) (end 35.56 19.558) (width 0.4064) (layer B.Cu) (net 12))
 (segment (start 61.722 23.876) (end 61.214 21.336) (width 0.8128) (layer B.Cu) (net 13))
 (segment (start 61.214 21.336) (end 54.356 20.828) (width 0.8128) (layer B.Cu) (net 13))
 (segment (start 54.356 29.21) (end 57.658 28.956) (width 0.8128) (layer B.Cu) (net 13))
 (segment (start 57.658 28.956) (end 60.198 27.94) (width 0.8128) (layer B.Cu) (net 13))
 (segment (start 60.198 27.94) (end 61.468 25.654) (width 0.8128) (layer B.Cu) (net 13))
 (segment (start 61.468 25.654) (end 61.722 23.876) (width 0.8128) (layer B.Cu) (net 13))
 (segment (start 54.356 26.67) (end 57.15 26.67) (width 0.8128) (layer B.Cu) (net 14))
 (segment (start 57.15 26.67) (end 58.42 23.876) (width 0.8128) (layer B.Cu) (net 14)))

